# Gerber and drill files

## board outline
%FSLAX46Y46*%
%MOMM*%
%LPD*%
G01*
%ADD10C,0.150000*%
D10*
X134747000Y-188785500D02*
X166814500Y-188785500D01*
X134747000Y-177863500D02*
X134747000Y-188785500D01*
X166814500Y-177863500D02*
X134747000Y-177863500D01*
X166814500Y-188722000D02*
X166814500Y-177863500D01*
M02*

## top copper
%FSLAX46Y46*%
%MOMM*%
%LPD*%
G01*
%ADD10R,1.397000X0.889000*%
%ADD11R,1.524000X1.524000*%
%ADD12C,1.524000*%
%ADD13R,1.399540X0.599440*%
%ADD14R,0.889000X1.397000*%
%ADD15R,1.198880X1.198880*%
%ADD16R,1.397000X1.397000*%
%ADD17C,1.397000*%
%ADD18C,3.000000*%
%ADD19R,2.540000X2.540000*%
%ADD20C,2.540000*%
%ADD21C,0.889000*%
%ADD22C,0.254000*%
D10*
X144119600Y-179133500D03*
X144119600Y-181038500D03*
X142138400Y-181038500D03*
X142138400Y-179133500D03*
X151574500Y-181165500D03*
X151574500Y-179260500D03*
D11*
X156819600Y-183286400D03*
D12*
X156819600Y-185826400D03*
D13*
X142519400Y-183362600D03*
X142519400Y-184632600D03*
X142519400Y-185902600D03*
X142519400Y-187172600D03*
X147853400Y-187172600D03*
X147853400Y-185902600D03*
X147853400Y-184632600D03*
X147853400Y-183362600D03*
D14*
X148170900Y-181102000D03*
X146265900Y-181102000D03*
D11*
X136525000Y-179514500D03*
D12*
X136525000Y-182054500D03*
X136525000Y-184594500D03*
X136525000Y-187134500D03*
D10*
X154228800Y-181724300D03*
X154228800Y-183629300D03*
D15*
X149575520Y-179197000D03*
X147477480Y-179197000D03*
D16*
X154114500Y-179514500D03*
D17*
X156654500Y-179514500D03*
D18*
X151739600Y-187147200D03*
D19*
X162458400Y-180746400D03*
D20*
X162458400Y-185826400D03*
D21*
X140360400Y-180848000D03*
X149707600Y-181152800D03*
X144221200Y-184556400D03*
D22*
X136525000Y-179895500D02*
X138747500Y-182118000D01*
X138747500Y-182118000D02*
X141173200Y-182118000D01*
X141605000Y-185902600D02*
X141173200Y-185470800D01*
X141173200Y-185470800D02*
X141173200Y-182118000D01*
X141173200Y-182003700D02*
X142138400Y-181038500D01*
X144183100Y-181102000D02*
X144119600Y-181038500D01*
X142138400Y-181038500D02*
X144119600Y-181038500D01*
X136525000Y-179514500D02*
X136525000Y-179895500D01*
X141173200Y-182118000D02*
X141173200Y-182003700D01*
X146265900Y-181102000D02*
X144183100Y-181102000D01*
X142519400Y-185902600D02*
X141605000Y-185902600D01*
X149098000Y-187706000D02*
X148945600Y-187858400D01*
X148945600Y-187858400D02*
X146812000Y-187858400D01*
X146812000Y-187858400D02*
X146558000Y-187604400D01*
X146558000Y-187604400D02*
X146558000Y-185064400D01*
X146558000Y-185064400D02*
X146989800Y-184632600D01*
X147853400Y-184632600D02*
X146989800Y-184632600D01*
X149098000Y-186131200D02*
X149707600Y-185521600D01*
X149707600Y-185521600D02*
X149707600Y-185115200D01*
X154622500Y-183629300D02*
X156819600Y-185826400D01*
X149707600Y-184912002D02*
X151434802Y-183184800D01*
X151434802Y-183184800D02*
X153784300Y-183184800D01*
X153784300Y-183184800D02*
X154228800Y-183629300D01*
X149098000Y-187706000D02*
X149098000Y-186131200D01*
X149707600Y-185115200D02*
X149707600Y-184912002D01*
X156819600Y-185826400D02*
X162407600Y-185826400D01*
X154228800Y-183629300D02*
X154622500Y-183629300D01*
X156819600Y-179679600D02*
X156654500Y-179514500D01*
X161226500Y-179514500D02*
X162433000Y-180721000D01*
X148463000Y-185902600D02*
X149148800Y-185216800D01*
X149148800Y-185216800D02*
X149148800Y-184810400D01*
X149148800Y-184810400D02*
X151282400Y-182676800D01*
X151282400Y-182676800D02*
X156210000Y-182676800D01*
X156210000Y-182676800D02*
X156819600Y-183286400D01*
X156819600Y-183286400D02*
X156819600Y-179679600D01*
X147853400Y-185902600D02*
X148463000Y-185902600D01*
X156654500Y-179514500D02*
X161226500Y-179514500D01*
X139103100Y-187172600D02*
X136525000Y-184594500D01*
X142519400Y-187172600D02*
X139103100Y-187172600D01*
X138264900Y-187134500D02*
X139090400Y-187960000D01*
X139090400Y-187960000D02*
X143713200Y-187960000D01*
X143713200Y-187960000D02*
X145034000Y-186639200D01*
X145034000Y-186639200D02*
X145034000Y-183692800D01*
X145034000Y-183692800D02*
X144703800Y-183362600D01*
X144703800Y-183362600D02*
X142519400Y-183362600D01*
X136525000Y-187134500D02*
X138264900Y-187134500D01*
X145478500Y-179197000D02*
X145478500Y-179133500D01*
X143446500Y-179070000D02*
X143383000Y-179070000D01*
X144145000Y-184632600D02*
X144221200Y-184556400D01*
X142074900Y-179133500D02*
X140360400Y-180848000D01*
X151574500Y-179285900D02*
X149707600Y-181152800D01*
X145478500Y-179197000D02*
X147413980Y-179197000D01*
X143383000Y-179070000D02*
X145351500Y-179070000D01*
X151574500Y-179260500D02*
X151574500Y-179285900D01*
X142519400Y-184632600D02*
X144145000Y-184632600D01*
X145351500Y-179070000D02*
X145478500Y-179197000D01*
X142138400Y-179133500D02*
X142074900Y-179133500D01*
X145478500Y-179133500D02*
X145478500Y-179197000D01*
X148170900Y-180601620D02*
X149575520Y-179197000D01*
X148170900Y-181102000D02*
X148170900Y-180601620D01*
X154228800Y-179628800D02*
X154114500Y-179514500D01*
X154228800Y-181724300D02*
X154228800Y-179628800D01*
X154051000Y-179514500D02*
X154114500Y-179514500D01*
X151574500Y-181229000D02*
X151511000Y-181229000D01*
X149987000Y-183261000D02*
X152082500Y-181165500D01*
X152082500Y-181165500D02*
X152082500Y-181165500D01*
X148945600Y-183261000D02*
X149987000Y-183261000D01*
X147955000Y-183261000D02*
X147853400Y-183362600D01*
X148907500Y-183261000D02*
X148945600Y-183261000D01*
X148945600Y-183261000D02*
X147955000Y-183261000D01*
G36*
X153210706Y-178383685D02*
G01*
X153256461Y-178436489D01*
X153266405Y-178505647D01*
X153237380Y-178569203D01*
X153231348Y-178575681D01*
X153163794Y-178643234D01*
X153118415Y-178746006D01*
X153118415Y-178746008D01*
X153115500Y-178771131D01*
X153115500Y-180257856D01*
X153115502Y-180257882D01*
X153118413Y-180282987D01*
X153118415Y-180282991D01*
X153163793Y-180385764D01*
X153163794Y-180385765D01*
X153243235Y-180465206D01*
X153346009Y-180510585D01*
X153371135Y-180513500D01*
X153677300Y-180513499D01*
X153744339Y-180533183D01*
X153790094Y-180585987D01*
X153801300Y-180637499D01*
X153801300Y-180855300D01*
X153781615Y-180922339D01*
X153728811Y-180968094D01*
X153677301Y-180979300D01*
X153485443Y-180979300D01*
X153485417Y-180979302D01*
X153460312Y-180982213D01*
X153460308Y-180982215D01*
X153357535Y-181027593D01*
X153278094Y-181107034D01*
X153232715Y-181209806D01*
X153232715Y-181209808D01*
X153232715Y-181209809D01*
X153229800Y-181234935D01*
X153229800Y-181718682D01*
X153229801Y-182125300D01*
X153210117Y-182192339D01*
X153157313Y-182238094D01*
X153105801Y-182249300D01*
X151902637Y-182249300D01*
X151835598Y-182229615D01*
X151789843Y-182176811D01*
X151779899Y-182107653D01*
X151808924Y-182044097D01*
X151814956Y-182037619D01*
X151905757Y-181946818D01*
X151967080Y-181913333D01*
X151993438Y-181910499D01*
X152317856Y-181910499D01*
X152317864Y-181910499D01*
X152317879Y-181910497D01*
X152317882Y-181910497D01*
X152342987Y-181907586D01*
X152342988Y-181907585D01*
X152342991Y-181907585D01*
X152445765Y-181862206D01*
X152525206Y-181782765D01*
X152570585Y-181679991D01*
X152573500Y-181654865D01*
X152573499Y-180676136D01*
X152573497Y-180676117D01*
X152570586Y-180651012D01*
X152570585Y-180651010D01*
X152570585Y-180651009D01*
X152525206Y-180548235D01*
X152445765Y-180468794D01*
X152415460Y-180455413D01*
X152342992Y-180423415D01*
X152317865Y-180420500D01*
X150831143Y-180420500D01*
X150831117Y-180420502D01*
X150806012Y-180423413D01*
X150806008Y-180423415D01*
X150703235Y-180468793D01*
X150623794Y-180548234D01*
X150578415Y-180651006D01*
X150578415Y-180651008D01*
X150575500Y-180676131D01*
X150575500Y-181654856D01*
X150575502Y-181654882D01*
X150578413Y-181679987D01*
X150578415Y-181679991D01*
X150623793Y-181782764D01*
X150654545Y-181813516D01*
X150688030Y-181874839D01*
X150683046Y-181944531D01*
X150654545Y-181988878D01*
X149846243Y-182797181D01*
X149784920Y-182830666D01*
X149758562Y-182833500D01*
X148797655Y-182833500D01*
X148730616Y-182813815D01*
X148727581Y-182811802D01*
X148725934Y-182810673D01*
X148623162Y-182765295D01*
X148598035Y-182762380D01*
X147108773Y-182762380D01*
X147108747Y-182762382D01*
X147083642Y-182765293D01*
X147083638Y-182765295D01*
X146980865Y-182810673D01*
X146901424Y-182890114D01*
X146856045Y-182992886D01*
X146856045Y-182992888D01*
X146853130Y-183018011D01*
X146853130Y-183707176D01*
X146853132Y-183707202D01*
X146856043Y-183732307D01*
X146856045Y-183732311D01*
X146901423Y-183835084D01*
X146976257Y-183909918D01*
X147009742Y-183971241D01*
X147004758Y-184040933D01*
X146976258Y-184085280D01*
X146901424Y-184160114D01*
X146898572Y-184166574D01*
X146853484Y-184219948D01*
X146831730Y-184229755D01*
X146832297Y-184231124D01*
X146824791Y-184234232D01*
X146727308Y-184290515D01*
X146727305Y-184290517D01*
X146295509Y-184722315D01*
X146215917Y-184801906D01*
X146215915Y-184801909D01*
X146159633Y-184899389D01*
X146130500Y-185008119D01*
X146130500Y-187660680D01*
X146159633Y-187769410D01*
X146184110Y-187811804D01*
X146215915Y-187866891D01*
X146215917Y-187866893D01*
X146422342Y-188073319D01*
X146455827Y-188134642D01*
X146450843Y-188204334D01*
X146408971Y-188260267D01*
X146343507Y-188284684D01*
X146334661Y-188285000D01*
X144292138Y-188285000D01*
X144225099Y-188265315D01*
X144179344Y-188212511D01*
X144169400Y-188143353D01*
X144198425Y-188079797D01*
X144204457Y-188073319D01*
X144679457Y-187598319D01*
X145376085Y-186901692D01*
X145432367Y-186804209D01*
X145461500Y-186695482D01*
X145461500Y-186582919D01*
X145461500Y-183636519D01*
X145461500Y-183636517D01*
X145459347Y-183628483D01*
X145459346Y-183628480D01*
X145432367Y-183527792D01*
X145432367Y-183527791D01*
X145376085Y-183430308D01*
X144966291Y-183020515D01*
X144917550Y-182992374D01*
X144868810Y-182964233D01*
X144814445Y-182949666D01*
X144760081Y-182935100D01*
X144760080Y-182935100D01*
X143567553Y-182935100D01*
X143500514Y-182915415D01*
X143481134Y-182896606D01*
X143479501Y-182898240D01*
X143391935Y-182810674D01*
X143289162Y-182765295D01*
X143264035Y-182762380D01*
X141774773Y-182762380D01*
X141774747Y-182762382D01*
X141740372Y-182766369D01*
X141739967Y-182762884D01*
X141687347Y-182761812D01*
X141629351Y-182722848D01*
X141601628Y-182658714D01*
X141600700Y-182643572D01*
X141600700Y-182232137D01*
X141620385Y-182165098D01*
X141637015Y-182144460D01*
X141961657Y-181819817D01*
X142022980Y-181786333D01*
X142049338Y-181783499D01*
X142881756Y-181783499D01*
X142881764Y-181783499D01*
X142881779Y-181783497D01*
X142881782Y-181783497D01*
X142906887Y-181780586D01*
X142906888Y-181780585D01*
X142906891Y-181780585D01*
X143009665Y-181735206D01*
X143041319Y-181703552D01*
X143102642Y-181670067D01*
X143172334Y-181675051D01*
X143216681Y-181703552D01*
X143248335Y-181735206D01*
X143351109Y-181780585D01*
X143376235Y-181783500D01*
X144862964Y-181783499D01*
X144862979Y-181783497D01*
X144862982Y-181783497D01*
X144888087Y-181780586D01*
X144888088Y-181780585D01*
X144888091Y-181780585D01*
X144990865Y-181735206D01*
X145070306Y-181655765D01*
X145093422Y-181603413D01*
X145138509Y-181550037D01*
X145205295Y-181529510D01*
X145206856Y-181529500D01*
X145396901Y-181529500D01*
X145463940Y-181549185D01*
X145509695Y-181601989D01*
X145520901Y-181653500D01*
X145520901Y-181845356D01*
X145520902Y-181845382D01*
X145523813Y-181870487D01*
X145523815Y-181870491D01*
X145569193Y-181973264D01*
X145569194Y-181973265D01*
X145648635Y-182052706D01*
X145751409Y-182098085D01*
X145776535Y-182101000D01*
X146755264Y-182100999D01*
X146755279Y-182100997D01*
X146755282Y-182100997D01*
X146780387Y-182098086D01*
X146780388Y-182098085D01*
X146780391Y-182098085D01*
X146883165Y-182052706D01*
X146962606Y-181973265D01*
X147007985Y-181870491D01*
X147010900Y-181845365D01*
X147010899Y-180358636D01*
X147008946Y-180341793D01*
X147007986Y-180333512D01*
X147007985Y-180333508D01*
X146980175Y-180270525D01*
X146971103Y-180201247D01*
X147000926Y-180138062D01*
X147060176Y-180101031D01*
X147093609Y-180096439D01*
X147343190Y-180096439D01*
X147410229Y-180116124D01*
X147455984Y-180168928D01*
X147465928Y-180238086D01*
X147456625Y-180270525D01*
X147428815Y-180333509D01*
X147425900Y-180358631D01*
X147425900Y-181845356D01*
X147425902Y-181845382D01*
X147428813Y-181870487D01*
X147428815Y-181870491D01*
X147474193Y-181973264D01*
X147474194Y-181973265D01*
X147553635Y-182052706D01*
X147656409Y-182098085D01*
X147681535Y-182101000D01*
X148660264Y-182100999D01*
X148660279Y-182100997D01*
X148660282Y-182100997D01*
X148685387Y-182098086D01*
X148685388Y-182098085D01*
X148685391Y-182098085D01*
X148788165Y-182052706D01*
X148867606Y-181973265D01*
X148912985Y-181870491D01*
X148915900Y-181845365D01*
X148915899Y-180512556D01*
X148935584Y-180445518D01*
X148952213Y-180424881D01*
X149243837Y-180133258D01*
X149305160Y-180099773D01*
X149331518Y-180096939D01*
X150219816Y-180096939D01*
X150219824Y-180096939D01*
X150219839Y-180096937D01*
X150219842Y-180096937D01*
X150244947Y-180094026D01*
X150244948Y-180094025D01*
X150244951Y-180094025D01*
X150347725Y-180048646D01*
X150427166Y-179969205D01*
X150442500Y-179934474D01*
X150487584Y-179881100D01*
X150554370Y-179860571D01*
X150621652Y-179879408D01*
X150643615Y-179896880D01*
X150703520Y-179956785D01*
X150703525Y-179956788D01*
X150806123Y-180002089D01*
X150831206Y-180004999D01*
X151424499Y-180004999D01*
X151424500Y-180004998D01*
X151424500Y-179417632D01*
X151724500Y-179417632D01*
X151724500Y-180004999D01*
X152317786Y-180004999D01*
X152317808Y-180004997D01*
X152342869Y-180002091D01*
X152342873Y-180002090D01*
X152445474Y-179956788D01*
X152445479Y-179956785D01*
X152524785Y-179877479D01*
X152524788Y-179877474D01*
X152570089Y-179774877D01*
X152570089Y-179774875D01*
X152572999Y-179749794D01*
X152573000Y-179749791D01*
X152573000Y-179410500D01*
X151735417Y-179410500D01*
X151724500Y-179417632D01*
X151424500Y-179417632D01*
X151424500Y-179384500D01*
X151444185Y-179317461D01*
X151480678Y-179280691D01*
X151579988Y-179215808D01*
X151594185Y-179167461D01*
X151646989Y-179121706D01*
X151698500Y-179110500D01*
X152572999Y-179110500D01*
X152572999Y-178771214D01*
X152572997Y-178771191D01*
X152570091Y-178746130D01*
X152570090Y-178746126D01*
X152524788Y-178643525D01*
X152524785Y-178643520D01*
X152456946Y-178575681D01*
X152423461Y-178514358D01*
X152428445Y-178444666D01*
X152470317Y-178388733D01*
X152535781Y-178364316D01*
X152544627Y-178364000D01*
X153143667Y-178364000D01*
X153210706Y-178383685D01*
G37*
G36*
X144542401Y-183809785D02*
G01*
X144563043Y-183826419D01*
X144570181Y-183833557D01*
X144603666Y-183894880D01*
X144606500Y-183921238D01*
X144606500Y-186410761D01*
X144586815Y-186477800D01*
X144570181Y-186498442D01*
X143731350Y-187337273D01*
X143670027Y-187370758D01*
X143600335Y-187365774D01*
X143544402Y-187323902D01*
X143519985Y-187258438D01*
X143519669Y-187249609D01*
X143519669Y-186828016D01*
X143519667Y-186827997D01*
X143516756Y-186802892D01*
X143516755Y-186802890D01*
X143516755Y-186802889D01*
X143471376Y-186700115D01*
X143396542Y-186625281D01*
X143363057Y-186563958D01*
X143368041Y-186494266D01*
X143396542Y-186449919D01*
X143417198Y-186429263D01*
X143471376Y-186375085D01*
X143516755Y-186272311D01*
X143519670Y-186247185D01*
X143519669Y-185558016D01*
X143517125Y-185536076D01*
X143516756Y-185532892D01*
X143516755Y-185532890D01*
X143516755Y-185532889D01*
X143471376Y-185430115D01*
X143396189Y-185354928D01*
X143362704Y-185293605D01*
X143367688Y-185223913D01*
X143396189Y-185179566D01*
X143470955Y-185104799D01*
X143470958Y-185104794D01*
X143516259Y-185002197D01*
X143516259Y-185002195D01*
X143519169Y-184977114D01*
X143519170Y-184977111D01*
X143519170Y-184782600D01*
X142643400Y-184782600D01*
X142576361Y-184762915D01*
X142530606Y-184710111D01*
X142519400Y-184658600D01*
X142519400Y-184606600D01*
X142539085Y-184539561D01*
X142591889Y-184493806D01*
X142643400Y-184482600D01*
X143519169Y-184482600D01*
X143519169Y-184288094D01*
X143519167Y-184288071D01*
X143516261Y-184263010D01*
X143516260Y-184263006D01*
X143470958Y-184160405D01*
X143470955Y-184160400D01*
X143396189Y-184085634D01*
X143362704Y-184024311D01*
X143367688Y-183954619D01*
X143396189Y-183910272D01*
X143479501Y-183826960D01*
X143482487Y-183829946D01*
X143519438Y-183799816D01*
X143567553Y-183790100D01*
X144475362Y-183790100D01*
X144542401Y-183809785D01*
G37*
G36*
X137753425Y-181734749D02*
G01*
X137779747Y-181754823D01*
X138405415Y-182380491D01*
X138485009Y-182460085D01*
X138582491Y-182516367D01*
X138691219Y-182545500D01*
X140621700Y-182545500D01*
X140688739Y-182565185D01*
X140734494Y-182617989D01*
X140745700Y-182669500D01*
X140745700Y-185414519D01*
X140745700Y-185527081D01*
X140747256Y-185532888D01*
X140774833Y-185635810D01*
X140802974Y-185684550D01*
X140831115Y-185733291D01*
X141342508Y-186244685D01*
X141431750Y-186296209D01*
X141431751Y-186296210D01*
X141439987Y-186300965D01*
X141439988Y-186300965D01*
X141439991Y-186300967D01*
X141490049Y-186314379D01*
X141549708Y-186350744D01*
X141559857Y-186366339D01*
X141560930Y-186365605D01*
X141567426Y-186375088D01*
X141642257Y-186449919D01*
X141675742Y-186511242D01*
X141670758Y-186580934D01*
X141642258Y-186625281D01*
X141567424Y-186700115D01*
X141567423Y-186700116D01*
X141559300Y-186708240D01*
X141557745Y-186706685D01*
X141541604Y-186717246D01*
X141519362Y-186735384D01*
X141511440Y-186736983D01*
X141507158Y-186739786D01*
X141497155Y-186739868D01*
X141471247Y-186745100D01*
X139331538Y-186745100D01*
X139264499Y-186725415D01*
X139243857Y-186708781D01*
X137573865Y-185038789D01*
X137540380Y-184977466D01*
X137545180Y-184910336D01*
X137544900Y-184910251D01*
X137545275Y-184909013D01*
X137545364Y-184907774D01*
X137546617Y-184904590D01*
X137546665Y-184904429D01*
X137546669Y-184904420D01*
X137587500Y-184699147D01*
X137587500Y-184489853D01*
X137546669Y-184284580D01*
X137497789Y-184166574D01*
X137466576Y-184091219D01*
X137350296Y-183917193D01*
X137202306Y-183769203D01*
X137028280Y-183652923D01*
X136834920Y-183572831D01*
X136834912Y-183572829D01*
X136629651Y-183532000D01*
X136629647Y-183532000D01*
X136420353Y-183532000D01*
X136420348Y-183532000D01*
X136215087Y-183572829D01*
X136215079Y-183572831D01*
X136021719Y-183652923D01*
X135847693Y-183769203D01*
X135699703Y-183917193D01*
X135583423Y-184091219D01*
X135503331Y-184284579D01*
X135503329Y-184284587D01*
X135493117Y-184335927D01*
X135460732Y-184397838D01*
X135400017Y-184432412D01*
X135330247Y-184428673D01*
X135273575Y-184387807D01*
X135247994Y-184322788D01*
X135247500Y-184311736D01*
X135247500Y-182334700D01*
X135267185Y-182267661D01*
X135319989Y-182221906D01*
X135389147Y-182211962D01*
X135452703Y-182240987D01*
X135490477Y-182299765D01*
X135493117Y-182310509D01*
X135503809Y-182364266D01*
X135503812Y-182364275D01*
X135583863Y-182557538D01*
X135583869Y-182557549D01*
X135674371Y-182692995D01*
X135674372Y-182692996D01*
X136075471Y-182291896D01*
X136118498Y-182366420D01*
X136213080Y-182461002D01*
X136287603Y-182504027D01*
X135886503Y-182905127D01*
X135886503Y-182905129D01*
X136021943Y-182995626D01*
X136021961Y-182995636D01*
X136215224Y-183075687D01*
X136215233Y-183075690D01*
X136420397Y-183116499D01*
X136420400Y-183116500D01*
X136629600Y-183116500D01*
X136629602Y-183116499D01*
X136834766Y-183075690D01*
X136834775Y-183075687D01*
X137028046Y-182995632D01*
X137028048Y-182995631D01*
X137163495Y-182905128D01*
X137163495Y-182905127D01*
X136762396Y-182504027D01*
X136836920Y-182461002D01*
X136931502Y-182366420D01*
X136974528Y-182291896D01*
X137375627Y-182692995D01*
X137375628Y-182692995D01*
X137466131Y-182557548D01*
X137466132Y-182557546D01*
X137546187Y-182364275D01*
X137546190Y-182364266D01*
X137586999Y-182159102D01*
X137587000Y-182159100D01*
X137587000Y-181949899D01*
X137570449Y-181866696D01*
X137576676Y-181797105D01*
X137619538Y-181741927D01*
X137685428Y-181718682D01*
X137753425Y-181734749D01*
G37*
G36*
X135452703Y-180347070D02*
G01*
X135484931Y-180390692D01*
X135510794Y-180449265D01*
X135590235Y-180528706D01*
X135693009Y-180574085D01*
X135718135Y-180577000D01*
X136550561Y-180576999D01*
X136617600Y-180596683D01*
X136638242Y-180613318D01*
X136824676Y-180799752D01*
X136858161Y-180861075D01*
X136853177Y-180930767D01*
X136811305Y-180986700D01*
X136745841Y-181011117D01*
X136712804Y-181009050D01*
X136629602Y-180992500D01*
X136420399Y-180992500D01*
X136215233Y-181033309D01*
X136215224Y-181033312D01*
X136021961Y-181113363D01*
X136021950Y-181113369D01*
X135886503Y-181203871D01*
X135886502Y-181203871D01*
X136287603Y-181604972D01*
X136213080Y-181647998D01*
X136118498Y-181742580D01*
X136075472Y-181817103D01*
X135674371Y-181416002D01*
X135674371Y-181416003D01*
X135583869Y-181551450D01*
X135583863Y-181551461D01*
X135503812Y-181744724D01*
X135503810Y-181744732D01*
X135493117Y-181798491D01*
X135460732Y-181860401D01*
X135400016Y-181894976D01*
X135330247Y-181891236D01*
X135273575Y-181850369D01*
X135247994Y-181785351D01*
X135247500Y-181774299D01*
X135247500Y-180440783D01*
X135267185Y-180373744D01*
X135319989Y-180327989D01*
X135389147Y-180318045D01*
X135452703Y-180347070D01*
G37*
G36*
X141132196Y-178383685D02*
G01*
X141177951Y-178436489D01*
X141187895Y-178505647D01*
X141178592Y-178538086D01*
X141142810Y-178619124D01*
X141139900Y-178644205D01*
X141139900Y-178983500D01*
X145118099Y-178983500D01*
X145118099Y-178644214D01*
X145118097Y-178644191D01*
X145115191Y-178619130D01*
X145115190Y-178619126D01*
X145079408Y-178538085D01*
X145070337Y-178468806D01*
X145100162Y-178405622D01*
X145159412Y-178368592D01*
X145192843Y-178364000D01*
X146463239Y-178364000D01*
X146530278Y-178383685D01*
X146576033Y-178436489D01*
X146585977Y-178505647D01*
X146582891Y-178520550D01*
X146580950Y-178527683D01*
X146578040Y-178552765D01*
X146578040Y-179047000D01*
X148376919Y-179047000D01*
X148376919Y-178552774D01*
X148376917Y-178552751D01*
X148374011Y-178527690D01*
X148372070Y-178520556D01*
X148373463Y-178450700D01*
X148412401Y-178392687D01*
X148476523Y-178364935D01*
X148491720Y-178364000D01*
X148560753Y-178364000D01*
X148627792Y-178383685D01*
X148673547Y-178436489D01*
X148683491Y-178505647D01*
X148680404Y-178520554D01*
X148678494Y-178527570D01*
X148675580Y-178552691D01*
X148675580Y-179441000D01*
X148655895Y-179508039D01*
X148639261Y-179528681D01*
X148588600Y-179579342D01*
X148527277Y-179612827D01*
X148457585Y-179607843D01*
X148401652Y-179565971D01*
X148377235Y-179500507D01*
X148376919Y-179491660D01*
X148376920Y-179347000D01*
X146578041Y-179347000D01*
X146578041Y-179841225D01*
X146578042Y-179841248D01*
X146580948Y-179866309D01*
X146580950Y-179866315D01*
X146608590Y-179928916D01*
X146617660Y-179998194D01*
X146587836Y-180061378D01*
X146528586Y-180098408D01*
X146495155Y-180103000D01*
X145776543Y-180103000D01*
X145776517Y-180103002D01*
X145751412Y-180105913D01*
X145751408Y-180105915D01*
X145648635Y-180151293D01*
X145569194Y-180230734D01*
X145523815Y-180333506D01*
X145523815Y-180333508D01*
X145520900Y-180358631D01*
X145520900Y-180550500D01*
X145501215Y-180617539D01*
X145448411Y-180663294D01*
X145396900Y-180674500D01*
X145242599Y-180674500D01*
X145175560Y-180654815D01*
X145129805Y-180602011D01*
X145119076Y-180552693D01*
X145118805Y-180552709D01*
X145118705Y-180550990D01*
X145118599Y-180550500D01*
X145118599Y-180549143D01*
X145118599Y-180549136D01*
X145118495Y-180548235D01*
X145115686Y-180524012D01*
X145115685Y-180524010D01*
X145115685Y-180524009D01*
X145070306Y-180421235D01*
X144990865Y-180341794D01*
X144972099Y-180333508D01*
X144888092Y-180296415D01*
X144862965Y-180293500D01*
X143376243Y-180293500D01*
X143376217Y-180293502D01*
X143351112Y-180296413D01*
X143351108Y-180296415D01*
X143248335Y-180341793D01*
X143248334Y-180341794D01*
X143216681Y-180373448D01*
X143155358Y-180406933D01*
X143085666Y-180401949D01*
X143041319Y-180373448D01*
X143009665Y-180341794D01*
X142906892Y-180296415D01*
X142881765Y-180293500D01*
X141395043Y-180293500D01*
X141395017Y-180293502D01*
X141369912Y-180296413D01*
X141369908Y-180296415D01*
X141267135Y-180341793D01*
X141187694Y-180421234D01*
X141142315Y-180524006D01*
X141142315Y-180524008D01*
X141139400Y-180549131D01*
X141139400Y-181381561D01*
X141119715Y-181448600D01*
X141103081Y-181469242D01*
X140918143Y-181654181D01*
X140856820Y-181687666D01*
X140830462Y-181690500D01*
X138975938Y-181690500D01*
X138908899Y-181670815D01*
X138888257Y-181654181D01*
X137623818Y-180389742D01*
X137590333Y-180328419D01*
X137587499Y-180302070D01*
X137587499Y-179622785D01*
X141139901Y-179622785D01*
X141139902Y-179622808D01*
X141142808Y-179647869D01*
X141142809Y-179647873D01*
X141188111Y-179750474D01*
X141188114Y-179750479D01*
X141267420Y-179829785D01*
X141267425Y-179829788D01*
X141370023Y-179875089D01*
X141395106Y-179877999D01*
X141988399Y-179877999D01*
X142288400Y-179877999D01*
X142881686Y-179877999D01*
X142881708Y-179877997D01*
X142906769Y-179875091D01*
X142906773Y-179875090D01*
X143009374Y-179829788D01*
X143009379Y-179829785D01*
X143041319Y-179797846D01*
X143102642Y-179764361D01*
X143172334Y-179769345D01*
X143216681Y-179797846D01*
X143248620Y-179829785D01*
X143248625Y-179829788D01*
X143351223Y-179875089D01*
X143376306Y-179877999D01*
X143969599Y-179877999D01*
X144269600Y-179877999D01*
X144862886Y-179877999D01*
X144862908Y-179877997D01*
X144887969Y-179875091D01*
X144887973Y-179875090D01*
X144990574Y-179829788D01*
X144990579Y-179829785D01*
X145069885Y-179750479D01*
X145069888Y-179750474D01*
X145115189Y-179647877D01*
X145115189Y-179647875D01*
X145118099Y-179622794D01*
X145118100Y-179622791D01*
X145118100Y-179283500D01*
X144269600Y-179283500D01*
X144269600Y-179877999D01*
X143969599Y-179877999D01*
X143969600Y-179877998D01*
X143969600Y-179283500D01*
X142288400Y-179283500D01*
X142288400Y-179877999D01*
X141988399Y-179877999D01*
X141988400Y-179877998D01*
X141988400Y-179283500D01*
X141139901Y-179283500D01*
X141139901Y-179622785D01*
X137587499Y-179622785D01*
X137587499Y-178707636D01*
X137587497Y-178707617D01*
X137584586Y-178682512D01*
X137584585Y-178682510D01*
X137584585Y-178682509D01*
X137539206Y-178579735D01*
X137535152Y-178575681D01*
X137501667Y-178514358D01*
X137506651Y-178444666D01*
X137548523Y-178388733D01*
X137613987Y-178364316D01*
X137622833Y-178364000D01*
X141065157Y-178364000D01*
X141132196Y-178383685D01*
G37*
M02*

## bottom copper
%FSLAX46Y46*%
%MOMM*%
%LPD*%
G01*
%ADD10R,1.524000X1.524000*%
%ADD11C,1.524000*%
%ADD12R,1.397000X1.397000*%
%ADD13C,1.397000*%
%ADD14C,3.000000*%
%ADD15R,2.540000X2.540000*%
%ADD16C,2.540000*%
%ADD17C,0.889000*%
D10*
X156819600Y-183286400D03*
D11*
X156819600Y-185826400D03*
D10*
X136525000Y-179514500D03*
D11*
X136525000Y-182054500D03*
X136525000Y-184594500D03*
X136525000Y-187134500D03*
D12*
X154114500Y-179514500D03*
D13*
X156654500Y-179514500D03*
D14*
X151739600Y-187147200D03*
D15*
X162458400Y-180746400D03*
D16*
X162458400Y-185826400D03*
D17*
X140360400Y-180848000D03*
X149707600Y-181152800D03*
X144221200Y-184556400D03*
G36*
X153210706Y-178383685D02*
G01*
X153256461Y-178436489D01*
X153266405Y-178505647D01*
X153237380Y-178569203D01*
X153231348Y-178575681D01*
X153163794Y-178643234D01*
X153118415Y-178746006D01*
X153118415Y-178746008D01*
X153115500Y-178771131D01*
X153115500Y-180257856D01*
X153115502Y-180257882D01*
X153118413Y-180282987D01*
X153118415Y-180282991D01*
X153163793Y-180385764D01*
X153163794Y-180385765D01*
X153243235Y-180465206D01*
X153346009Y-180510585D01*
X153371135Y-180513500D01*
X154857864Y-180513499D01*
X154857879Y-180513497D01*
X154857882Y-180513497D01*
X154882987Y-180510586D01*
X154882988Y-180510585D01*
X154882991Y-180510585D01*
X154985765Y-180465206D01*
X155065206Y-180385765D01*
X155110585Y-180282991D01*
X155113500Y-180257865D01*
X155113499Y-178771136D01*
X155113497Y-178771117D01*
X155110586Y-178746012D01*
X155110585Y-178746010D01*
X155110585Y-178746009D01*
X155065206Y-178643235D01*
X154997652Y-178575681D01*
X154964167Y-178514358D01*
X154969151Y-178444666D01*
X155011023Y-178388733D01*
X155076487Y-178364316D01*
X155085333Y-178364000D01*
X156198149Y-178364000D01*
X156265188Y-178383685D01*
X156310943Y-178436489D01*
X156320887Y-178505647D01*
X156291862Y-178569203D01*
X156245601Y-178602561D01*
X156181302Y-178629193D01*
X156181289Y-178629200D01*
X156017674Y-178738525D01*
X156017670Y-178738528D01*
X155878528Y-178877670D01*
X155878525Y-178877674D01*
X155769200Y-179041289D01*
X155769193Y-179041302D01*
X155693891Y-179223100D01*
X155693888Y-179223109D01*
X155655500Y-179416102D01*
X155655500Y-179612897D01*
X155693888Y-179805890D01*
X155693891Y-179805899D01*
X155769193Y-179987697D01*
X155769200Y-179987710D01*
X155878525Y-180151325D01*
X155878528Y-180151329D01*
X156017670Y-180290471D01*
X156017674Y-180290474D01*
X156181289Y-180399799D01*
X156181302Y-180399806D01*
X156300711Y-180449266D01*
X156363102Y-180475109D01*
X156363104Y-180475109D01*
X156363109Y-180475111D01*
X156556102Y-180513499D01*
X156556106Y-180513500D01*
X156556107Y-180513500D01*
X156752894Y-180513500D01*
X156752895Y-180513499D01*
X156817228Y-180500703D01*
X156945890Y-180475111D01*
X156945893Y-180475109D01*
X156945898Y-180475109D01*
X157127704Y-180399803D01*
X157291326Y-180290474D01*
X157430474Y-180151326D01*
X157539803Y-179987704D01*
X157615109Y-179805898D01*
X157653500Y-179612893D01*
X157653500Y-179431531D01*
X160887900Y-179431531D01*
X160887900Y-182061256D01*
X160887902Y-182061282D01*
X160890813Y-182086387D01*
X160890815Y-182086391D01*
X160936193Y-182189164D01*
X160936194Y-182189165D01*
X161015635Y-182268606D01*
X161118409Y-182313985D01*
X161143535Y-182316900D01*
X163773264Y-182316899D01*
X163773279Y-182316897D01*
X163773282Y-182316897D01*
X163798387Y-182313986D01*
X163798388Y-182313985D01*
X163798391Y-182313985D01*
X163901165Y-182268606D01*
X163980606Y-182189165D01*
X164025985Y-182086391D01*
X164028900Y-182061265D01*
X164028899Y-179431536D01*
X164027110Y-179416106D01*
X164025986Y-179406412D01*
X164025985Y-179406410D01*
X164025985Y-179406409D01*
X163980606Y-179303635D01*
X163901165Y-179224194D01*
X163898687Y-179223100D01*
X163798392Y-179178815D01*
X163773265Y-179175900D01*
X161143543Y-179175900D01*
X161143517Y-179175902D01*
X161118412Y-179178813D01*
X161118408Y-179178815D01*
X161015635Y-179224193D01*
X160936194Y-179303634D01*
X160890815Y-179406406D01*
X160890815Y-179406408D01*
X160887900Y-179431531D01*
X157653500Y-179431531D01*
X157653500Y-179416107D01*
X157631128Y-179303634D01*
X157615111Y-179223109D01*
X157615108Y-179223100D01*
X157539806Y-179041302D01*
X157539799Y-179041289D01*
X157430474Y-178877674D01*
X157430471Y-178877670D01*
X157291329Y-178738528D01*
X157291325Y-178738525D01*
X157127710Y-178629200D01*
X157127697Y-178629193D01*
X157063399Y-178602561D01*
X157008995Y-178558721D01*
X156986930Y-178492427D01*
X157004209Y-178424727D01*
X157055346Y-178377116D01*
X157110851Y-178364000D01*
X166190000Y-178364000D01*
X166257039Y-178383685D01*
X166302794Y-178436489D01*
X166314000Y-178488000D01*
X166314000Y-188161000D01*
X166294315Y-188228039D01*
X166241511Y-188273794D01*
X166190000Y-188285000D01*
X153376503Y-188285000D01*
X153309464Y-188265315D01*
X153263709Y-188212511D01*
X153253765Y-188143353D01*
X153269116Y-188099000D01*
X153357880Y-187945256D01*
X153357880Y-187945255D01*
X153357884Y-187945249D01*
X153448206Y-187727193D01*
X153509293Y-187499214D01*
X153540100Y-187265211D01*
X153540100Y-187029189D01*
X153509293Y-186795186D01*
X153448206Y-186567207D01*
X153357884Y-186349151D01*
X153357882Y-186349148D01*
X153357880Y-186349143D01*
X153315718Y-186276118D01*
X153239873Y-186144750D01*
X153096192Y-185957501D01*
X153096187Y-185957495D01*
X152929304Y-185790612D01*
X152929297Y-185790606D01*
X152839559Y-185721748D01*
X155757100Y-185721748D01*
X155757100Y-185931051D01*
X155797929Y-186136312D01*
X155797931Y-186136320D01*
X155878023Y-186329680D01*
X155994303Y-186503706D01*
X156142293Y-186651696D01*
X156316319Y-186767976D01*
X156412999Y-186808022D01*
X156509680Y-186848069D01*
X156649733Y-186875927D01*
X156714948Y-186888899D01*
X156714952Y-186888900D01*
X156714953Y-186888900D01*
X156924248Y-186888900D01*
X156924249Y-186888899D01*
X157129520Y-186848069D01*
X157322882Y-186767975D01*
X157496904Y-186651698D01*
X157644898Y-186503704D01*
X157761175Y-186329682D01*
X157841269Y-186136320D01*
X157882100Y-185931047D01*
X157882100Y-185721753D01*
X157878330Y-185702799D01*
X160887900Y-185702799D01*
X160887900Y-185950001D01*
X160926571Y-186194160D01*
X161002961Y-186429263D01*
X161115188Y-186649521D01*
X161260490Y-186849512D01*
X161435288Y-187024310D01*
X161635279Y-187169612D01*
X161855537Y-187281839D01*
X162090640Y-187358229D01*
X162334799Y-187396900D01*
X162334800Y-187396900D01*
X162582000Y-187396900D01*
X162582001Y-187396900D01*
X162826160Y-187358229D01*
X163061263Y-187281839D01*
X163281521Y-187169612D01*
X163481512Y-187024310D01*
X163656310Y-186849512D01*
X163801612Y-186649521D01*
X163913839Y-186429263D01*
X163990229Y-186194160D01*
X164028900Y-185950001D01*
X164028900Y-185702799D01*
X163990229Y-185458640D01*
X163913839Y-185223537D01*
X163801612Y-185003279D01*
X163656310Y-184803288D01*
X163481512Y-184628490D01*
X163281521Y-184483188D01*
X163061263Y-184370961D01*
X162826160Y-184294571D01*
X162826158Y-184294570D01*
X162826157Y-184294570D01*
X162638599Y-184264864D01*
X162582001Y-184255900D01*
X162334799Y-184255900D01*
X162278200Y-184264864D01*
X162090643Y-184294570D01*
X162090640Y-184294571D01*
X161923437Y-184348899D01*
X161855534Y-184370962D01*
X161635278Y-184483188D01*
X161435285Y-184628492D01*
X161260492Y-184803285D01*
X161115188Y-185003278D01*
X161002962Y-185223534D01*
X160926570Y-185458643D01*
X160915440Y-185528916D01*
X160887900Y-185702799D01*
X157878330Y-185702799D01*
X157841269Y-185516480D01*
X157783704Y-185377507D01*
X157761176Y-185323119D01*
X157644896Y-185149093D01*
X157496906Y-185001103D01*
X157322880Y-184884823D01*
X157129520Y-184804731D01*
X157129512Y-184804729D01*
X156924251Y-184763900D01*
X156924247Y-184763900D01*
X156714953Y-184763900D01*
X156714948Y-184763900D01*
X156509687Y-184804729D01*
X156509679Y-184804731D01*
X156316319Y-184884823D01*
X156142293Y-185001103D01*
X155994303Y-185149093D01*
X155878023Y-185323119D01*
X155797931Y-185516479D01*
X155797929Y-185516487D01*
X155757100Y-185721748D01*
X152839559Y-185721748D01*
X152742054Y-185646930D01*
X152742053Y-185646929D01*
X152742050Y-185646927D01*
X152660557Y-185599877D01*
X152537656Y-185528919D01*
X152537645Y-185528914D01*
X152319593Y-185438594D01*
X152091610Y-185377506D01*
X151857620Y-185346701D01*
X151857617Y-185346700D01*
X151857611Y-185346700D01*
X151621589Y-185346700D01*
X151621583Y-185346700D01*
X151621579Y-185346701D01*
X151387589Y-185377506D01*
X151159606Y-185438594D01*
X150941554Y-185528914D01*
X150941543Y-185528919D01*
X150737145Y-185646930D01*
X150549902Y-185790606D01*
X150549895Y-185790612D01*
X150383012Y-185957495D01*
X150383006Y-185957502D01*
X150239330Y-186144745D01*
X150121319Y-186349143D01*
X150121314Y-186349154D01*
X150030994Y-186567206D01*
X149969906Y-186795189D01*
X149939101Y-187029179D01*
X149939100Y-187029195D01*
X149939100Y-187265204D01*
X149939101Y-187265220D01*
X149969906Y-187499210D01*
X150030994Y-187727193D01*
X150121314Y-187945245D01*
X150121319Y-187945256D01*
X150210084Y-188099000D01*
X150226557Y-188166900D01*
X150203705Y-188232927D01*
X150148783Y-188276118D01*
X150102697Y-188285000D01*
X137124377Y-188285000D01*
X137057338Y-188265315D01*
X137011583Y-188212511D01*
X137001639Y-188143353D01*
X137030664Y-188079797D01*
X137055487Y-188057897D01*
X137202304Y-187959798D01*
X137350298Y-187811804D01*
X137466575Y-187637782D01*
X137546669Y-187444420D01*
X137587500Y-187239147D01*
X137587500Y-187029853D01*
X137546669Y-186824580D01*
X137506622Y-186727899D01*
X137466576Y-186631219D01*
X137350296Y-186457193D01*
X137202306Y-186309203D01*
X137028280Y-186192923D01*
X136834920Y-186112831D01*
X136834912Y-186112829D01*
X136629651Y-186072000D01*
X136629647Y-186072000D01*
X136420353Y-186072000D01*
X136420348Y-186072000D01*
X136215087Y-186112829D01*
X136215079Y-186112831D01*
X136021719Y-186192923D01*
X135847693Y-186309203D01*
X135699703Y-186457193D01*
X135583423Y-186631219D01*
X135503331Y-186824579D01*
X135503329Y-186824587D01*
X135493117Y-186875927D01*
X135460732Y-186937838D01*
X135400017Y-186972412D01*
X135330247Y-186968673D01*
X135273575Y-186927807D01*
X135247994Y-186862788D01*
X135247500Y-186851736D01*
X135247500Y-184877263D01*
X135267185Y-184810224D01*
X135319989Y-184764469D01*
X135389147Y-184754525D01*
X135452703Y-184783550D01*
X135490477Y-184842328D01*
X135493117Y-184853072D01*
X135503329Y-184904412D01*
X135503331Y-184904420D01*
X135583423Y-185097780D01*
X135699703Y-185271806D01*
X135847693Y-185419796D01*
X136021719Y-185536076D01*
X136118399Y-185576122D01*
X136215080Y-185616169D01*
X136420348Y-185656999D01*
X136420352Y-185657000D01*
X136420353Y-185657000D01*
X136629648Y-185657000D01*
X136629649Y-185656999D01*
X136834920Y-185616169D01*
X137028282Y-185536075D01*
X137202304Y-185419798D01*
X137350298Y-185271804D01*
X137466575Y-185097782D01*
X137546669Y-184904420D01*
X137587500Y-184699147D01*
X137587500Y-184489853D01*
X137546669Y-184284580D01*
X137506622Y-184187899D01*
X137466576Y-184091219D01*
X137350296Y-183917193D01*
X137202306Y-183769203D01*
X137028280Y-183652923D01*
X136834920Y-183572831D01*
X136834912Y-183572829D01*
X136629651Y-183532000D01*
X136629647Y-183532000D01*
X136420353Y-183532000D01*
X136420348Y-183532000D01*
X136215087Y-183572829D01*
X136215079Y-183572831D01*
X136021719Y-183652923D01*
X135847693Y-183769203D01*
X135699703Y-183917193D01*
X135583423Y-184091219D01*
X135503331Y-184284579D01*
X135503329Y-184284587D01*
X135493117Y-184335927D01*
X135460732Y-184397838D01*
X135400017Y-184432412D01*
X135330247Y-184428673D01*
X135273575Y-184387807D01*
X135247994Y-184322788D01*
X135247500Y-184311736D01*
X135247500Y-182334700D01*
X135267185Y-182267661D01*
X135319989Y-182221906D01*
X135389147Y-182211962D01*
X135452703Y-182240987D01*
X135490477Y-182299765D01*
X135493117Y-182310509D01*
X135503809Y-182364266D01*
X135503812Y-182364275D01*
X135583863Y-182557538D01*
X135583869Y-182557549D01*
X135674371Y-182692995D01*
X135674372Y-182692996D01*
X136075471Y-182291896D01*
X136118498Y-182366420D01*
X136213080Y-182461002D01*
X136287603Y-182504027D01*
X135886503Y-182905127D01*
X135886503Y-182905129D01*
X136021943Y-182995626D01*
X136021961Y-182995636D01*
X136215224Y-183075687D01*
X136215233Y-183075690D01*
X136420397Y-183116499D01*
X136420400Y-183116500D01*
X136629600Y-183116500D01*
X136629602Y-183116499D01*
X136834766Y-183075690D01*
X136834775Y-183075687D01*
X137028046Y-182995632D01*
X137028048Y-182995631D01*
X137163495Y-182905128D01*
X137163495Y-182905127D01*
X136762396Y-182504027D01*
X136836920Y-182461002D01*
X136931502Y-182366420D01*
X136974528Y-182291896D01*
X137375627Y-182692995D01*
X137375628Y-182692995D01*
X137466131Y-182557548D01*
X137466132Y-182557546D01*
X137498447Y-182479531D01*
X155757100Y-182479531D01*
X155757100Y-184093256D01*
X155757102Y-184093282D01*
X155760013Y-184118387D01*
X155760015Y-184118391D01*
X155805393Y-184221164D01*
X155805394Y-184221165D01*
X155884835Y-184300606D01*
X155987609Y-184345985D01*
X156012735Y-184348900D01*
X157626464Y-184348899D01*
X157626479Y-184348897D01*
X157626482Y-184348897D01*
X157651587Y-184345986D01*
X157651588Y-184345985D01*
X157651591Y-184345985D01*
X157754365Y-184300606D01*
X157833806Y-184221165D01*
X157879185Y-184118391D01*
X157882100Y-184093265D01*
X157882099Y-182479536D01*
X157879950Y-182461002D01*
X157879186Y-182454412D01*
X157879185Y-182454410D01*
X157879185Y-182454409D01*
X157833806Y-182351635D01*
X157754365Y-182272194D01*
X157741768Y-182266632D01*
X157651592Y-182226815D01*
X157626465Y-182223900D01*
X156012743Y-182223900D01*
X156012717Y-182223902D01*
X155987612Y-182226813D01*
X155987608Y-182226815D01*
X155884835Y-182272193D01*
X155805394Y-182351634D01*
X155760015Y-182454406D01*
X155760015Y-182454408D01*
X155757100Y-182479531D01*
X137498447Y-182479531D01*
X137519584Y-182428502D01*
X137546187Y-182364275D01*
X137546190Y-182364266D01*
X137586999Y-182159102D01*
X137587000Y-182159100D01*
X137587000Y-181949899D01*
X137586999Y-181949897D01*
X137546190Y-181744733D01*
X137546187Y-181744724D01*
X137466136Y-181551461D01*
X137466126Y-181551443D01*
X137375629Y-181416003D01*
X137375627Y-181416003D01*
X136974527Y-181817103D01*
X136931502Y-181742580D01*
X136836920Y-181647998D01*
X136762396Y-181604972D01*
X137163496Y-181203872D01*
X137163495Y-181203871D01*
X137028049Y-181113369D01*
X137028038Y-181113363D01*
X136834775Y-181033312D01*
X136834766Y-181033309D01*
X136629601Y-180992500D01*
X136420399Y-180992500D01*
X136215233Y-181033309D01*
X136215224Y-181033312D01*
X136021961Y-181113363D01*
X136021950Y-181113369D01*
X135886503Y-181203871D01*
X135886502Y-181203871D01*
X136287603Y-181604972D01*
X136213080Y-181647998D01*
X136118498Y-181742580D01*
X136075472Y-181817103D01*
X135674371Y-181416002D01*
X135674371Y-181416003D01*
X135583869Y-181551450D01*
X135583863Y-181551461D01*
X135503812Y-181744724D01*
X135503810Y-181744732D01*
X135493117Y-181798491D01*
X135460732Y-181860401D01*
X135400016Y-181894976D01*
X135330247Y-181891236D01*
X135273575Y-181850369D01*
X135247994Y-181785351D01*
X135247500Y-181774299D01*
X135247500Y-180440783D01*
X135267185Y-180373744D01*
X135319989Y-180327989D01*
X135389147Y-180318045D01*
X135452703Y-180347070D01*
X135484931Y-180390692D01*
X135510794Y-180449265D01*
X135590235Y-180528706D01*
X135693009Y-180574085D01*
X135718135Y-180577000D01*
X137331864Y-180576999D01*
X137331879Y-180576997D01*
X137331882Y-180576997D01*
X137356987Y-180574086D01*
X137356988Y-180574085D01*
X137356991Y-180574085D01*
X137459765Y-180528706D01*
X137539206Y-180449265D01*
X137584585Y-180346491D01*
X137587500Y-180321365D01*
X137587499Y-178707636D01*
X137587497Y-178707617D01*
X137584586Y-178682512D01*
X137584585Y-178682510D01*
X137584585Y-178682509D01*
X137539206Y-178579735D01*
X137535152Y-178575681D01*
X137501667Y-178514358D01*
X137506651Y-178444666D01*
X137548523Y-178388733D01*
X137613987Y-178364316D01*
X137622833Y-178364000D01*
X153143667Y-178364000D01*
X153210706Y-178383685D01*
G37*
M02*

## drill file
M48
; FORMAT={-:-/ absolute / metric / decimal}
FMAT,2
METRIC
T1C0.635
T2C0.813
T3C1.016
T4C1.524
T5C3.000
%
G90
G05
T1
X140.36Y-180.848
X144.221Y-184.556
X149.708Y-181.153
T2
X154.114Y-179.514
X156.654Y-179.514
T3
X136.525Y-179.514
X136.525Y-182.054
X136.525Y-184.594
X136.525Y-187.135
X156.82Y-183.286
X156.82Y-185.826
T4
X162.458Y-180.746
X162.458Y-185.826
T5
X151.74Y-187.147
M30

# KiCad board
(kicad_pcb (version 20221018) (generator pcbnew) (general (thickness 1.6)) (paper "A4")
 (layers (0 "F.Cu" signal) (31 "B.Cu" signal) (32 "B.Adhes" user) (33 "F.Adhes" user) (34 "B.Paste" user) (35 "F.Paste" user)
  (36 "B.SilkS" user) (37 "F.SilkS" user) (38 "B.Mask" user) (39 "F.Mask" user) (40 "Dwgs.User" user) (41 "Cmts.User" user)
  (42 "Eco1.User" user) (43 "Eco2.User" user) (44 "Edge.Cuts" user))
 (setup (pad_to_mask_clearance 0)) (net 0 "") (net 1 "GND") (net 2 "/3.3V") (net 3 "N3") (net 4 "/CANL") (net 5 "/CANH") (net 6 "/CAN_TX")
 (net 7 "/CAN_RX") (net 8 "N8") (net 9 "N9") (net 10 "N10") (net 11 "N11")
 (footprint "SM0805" (layer "F.Cu") (at 144.1196 180.086 -90)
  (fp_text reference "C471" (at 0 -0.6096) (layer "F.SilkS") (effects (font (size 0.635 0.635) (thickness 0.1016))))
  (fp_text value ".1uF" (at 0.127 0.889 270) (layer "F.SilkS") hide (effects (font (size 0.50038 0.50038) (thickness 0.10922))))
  (pad "1" smd rect (at -0.9525 0 270) (size 0.889 1.397) (layers "F.Cu" "F.Paste" "F.Mask") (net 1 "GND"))
  (pad "2" smd rect (at 0.9525 0 270) (size 0.889 1.397) (layers "F.Cu" "F.Paste" "F.Mask") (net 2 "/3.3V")))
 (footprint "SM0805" (layer "F.Cu") (at 142.1384 180.086 90)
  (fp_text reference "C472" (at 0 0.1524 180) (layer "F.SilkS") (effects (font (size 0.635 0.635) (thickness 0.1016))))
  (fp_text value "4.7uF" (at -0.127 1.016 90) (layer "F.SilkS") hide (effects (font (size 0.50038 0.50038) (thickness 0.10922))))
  (pad "1" smd rect (at -0.9525 0 90) (size 0.889 1.397) (layers "F.Cu" "F.Paste" "F.Mask") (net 2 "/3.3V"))
  (pad "2" smd rect (at 0.9525 0 90) (size 0.889 1.397) (layers "F.Cu" "F.Paste" "F.Mask") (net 1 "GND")))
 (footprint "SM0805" (layer "F.Cu") (at 151.5745 180.213 90)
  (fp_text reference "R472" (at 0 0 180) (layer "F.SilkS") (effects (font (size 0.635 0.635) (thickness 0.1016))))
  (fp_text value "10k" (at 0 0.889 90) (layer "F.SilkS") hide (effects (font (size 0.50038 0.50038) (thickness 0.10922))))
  (pad "1" smd rect (at -0.9525 0 90) (size 0.889 1.397) (layers "F.Cu" "F.Paste" "F.Mask") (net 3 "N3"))
  (pad "2" smd rect (at 0.9525 0 90) (size 0.889 1.397) (layers "F.Cu" "F.Paste" "F.Mask") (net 1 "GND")))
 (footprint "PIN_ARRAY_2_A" (layer "F.Cu") (at 156.8196 184.5564 -90)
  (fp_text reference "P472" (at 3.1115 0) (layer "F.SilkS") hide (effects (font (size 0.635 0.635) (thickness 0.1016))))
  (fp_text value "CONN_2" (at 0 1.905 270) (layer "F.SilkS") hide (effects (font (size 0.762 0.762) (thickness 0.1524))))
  (pad "1" thru_hole rect (at -1.27 0 270) (size 1.524 1.524) (drill 1.016) (layers "*.Cu" "*.Mask" "F.SilkS") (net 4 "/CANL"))
  (pad "2" thru_hole circle (at 1.27 0 270) (size 1.524 1.524) (drill 1.016) (layers "*.Cu" "*.Mask" "F.SilkS") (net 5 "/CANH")))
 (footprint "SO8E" (layer "F.Cu") (at 145.1864 185.2676 -90)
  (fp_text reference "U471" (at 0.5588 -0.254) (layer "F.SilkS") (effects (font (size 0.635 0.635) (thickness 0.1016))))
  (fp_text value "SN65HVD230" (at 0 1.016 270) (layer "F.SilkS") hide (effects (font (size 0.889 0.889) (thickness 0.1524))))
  (pad "1" smd rect (at -1.905 2.667 270) (size 0.59944 1.39954) (layers "F.Cu" "F.Paste" "F.Mask") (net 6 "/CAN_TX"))
  (pad "2" smd rect (at -0.635 2.667 270) (size 0.59944 1.39954) (layers "F.Cu" "F.Paste" "F.Mask") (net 1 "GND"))
  (pad "3" smd rect (at 0.635 2.667 270) (size 0.59944 1.39954) (layers "F.Cu" "F.Paste" "F.Mask") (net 2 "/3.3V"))
  (pad "4" smd rect (at 1.905 2.667 270) (size 0.59944 1.39954) (layers "F.Cu" "F.Paste" "F.Mask") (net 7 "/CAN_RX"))
  (pad "5" smd rect (at 1.905 -2.667 270) (size 0.59944 1.39954) (layers "F.Cu" "F.Paste" "F.Mask") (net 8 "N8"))
  (pad "6" smd rect (at 0.635 -2.667 270) (size 0.59944 1.39954) (layers "F.Cu" "F.Paste" "F.Mask") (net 4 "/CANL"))
  (pad "7" smd rect (at -0.635 -2.667 270) (size 0.59944 1.39954) (layers "F.Cu" "F.Paste" "F.Mask") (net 5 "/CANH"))
  (pad "8" smd rect (at -1.905 -2.667 270) (size 0.59944 1.39954) (layers "F.Cu" "F.Paste" "F.Mask") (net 3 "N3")))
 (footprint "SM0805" (layer "F.Cu") (at 147.2184 181.102 180)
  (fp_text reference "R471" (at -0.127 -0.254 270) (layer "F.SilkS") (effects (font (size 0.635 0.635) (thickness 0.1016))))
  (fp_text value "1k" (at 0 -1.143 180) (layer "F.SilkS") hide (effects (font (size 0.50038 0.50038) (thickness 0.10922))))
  (pad "1" smd rect (at -0.9525 0 180) (size 0.889 1.397) (layers "F.Cu" "F.Paste" "F.Mask") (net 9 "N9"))
  (pad "2" smd rect (at 0.9525 0 180) (size 0.889 1.397) (layers "F.Cu" "F.Paste" "F.Mask") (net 2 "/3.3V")))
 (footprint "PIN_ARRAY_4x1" (layer "F.Cu") (at 136.525 183.3245 -90)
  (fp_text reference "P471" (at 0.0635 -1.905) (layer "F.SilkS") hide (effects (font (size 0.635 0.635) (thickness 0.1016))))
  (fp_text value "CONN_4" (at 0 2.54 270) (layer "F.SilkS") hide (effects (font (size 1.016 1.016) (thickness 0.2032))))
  (pad "1" thru_hole rect (at -3.81 0 270) (size 1.524 1.524) (drill 1.016) (layers "*.Cu" "*.Mask" "F.SilkS") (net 2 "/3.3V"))
  (pad "2" thru_hole circle (at -1.27 0 270) (size 1.524 1.524) (drill 1.016) (layers "*.Cu" "*.Mask" "F.SilkS") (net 1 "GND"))
  (pad "3" thru_hole circle (at 1.27 0 270) (size 1.524 1.524) (drill 1.016) (layers "*.Cu" "*.Mask" "F.SilkS") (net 7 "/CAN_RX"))
  (pad "4" thru_hole circle (at 3.81 0 270) (size 1.524 1.524) (drill 1.016) (layers "*.Cu" "*.Mask" "F.SilkS") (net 6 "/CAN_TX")))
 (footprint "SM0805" (layer "F.Cu") (at 154.2288 182.6768 -90)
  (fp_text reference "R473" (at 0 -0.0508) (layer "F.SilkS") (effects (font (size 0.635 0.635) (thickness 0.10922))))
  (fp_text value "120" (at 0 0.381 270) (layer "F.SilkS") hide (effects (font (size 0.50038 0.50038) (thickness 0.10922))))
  (pad "1" smd rect (at -0.9525 0 270) (size 0.889 1.397) (layers "F.Cu" "F.Paste" "F.Mask") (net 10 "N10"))
  (pad "2" smd rect (at 0.9525 0 270) (size 0.889 1.397) (layers "F.Cu" "F.Paste" "F.Mask") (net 5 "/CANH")))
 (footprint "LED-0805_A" (layer "F.Cu") (at 148.5265 179.197 180)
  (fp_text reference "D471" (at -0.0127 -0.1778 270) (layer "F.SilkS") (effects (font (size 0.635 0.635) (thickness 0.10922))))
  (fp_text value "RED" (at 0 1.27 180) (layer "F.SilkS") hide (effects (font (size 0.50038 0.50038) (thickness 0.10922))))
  (pad "1" smd rect (at -1.04902 0 180) (size 1.19888 1.19888) (layers "F.Cu" "F.Paste" "F.Mask") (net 9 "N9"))
  (pad "2" smd rect (at 1.04902 0 180) (size 1.19888 1.19888) (layers "F.Cu" "F.Paste" "F.Mask") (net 1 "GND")))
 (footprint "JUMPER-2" (layer "F.Cu") (at 155.3845 179.5145)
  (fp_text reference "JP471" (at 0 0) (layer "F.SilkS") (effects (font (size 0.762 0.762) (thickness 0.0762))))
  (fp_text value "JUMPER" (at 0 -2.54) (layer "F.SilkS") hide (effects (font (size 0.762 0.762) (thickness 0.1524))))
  (pad "1" thru_hole rect (at -1.27 0) (size 1.397 1.397) (drill 0.8128) (layers "*.Cu" "*.Mask" "F.SilkS") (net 10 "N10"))
  (pad "2" thru_hole circle (at 1.27 0) (size 1.397 1.397) (drill 0.8128) (layers "*.Cu" "*.Mask" "F.SilkS") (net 4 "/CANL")))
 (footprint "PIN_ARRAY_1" (layer "F.Cu") (at 151.7396 187.1472)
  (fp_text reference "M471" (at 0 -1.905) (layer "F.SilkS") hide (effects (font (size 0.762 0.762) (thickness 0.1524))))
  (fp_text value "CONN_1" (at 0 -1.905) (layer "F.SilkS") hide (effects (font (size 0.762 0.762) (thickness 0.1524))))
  (pad "1" thru_hole circle (at 0 0) (size 3 3) (drill 3) (layers "*.Cu" "*.Mask" "F.SilkS") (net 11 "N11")))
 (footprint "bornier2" (layer "F.Cu") (at 162.4584 183.2864 -90)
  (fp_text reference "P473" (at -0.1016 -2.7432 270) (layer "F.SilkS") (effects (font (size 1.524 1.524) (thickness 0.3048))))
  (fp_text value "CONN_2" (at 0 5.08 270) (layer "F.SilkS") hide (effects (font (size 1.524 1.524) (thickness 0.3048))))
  (pad "1" thru_hole rect (at -2.54 0 270) (size 2.54 2.54) (drill 1.524) (layers "*.Cu" "*.Mask" "F.SilkS") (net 4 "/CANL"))
  (pad "2" thru_hole circle (at 2.54 0 270) (size 2.54 2.54) (drill 1.524) (layers "*.Cu" "*.Mask" "F.SilkS") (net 5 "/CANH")))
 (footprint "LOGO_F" (layer "B.Cu") (at 146.4564 182.7784)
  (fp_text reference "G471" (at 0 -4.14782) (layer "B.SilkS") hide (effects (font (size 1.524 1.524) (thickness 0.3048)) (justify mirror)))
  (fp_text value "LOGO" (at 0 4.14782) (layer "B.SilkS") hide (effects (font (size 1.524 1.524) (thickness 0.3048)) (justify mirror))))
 (gr_line (start 134.747 188.7855) (end 166.8145 188.7855) (stroke (width 0.15) (type solid)) (layer "Edge.Cuts"))
 (gr_line (start 134.747 177.8635) (end 134.747 188.7855) (stroke (width 0.15) (type solid)) (layer "Edge.Cuts"))
 (gr_line (start 166.8145 177.8635) (end 134.747 177.8635) (stroke (width 0.15) (type solid)) (layer "Edge.Cuts"))
 (gr_line (start 166.8145 188.722) (end 166.8145 177.8635) (stroke (width 0.15) (type solid)) (layer "Edge.Cuts"))
 (segment (start 136.525 179.8955) (end 138.7475 182.118) (width 0.254) (layer "F.Cu") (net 2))
 (segment (start 138.7475 182.118) (end 141.1732 182.118) (width 0.254) (layer "F.Cu") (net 2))
 (segment (start 141.605 185.9026) (end 141.1732 185.4708) (width 0.254) (layer "F.Cu") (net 2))
 (segment (start 141.1732 185.4708) (end 141.1732 182.118) (width 0.254) (layer "F.Cu") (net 2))
 (segment (start 141.1732 182.0037) (end 142.1384 181.0385) (width 0.254) (layer "F.Cu") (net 2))
 (segment (start 144.1831 181.102) (end 144.1196 181.0385) (width 0.254) (layer "F.Cu") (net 2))
 (segment (start 142.1384 181.0385) (end 144.1196 181.0385) (width 0.254) (layer "F.Cu") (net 2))
 (segment (start 136.525 179.5145) (end 136.525 179.8955) (width 0.254) (layer "F.Cu") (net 2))
 (segment (start 141.1732 182.118) (end 141.1732 182.0037) (width 0.254) (layer "F.Cu") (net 2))
 (segment (start 146.2659 181.102) (end 144.1831 181.102) (width 0.254) (layer "F.Cu") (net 2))
 (segment (start 142.5194 185.9026) (end 141.605 185.9026) (width 0.254) (layer "F.Cu") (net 2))
 (segment (start 149.098 187.706) (end 148.9456 187.8584) (width 0.254) (layer "F.Cu") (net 5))
 (segment (start 148.9456 187.8584) (end 146.812 187.8584) (width 0.254) (layer "F.Cu") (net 5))
 (segment (start 146.812 187.8584) (end 146.558 187.6044) (width 0.254) (layer "F.Cu") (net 5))
 (segment (start 146.558 187.6044) (end 146.558 185.0644) (width 0.254) (layer "F.Cu") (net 5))
 (segment (start 146.558 185.0644) (end 146.9898 184.6326) (width 0.254) (layer "F.Cu") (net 5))
 (segment (start 147.8534 184.6326) (end 146.9898 184.6326) (width 0.254) (layer "F.Cu") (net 5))
 (segment (start 149.098 186.1312) (end 149.7076 185.5216) (width 0.254) (layer "F.Cu") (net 5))
 (segment (start 149.7076 185.5216) (end 149.7076 185.1152) (width 0.254) (layer "F.Cu") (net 5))
 (segment (start 154.6225 183.6293) (end 156.8196 185.8264) (width 0.254) (layer "F.Cu") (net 5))
 (segment (start 149.7076 184.912002) (end 151.434802 183.1848) (width 0.254) (layer "F.Cu") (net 5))
 (segment (start 151.434802 183.1848) (end 153.7843 183.1848) (width 0.254) (layer "F.Cu") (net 5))
 (segment (start 153.7843 183.1848) (end 154.2288 183.6293) (width 0.254) (layer "F.Cu") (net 5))
 (segment (start 149.098 187.706) (end 149.098 186.1312) (width 0.254) (layer "F.Cu") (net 5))
 (segment (start 149.7076 185.1152) (end 149.7076 184.912002) (width 0.254) (layer "F.Cu") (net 5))
 (segment (start 156.8196 185.8264) (end 162.4076 185.8264) (width 0.254) (layer "F.Cu") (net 5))
 (segment (start 154.2288 183.6293) (end 154.6225 183.6293) (width 0.254) (layer "F.Cu") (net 5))
 (segment (start 156.8196 179.6796) (end 156.6545 179.5145) (width 0.254) (layer "F.Cu") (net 4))
 (segment (start 161.2265 179.5145) (end 162.433 180.721) (width 0.254) (layer "F.Cu") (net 4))
 (segment (start 148.463 185.9026) (end 149.1488 185.2168) (width 0.254) (layer "F.Cu") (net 4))
 (segment (start 149.1488 185.2168) (end 149.1488 184.8104) (width 0.254) (layer "F.Cu") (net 4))
 (segment (start 149.1488 184.8104) (end 151.2824 182.6768) (width 0.254) (layer "F.Cu") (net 4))
 (segment (start 151.2824 182.6768) (end 156.21 182.6768) (width 0.254) (layer "F.Cu") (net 4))
 (segment (start 156.21 182.6768) (end 156.8196 183.2864) (width 0.254) (layer "F.Cu") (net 4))
 (segment (start 156.8196 183.2864) (end 156.8196 179.6796) (width 0.254) (layer "F.Cu") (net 4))
 (segment (start 147.8534 185.9026) (end 148.463 185.9026) (width 0.254) (layer "F.Cu") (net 4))
 (segment (start 156.6545 179.5145) (end 161.2265 179.5145) (width 0.254) (layer "F.Cu") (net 4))
 (segment (start 139.1031 187.1726) (end 136.525 184.5945) (width 0.254) (layer "F.Cu") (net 7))
 (segment (start 142.5194 187.1726) (end 139.1031 187.1726) (width 0.254) (layer "F.Cu") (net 7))
 (segment (start 138.2649 187.1345) (end 139.0904 187.96) (width 0.254) (layer "F.Cu") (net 6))
 (segment (start 139.0904 187.96) (end 143.7132 187.96) (width 0.254) (layer "F.Cu") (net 6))
 (segment (start 143.7132 187.96) (end 145.034 186.6392) (width 0.254) (layer "F.Cu") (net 6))
 (segment (start 145.034 186.6392) (end 145.034 183.6928) (width 0.254) (layer "F.Cu") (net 6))
 (segment (start 145.034 183.6928) (end 144.7038 183.3626) (width 0.254) (layer "F.Cu") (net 6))
 (segment (start 144.7038 183.3626) (end 142.5194 183.3626) (width 0.254) (layer "F.Cu") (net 6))
 (segment (start 136.525 187.1345) (end 138.2649 187.1345) (width 0.254) (layer "F.Cu") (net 6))
 (segment (start 145.4785 179.197) (end 145.4785 179.1335) (width 0.254) (layer "F.Cu") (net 1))
 (segment (start 143.4465 179.07) (end 143.383 179.07) (width 0.254) (layer "F.Cu") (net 1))
 (segment (start 144.145 184.6326) (end 144.2212 184.5564) (width 0.254) (layer "F.Cu") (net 1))
 (segment (start 142.0749 179.1335) (end 140.3604 180.848) (width 0.254) (layer "F.Cu") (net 1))
 (segment (start 151.5745 179.2859) (end 149.7076 181.1528) (width 0.254) (layer "F.Cu") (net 1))
 (segment (start 145.4785 179.197) (end 147.41398 179.197) (width 0.254) (layer "F.Cu") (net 1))
 (segment (start 143.383 179.07) (end 145.3515 179.07) (width 0.254) (layer "F.Cu") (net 1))
 (segment (start 151.5745 179.2605) (end 151.5745 179.2859) (width 0.254) (layer "F.Cu") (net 1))
 (segment (start 142.5194 184.6326) (end 144.145 184.6326) (width 0.254) (layer "F.Cu") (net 1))
 (segment (start 145.3515 179.07) (end 145.4785 179.197) (width 0.254) (layer "F.Cu") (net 1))
 (segment (start 142.1384 179.1335) (end 142.0749 179.1335) (width 0.254) (layer "F.Cu") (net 1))
 (segment (start 145.4785 179.1335) (end 145.4785 179.197) (width 0.254) (layer "F.Cu") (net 1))
 (via (at 140.3604 180.848) (size 0.889) (drill 0.635) (layers "F.Cu" "B.Cu") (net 1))
 (via (at 149.7076 181.1528) (size 0.889) (drill 0.635) (layers "F.Cu" "B.Cu") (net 1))
 (via (at 144.2212 184.5564) (size 0.889) (drill 0.635) (layers "F.Cu" "B.Cu") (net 1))
 (segment (start 148.1709 180.60162) (end 149.57552 179.197) (width 0.254) (layer "F.Cu") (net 9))
 (segment (start 148.1709 181.102) (end 148.1709 180.60162) (width 0.254) (layer "F.Cu") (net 9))
 (segment (start 154.2288 179.6288) (end 154.1145 179.5145) (width 0.254) (layer "F.Cu") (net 10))
 (segment (start 154.2288 181.7243) (end 154.2288 179.6288) (width 0.254) (layer "F.Cu") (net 10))
 (segment (start 154.051 179.5145) (end 154.1145 179.5145) (width 0.254) (layer "F.Cu") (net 10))
 (segment (start 151.5745 181.229) (end 151.511 181.229) (width 0.254) (layer "F.Cu") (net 3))
 (segment (start 149.987 183.261) (end 152.0825 181.1655) (width 0.254) (layer "F.Cu") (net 3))
 (segment (start 152.0825 181.1655) (end 152.0825 181.1655) (width 0.254) (layer "F.Cu") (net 3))
 (segment (start 148.9456 183.261) (end 149.987 183.261) (width 0.254) (layer "F.Cu") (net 3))
 (segment (start 147.955 183.261) (end 147.8534 183.3626) (width 0.254) (layer "F.Cu") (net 3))
 (segment (start 148.9075 183.261) (end 148.9456 183.261) (width 0.254) (layer "F.Cu") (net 3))
 (segment (start 148.9456 183.261) (end 147.955 183.261) (width 0.254) (layer "F.Cu") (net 3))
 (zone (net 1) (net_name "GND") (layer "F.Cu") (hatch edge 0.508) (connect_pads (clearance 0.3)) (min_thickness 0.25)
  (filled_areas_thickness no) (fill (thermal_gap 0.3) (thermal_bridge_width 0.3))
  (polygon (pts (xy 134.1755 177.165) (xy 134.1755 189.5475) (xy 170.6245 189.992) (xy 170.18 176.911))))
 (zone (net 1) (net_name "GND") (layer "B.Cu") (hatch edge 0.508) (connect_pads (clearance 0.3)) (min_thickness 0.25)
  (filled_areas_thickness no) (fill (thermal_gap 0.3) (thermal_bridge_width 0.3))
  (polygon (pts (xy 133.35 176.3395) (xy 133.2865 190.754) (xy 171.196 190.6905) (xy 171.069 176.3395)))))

